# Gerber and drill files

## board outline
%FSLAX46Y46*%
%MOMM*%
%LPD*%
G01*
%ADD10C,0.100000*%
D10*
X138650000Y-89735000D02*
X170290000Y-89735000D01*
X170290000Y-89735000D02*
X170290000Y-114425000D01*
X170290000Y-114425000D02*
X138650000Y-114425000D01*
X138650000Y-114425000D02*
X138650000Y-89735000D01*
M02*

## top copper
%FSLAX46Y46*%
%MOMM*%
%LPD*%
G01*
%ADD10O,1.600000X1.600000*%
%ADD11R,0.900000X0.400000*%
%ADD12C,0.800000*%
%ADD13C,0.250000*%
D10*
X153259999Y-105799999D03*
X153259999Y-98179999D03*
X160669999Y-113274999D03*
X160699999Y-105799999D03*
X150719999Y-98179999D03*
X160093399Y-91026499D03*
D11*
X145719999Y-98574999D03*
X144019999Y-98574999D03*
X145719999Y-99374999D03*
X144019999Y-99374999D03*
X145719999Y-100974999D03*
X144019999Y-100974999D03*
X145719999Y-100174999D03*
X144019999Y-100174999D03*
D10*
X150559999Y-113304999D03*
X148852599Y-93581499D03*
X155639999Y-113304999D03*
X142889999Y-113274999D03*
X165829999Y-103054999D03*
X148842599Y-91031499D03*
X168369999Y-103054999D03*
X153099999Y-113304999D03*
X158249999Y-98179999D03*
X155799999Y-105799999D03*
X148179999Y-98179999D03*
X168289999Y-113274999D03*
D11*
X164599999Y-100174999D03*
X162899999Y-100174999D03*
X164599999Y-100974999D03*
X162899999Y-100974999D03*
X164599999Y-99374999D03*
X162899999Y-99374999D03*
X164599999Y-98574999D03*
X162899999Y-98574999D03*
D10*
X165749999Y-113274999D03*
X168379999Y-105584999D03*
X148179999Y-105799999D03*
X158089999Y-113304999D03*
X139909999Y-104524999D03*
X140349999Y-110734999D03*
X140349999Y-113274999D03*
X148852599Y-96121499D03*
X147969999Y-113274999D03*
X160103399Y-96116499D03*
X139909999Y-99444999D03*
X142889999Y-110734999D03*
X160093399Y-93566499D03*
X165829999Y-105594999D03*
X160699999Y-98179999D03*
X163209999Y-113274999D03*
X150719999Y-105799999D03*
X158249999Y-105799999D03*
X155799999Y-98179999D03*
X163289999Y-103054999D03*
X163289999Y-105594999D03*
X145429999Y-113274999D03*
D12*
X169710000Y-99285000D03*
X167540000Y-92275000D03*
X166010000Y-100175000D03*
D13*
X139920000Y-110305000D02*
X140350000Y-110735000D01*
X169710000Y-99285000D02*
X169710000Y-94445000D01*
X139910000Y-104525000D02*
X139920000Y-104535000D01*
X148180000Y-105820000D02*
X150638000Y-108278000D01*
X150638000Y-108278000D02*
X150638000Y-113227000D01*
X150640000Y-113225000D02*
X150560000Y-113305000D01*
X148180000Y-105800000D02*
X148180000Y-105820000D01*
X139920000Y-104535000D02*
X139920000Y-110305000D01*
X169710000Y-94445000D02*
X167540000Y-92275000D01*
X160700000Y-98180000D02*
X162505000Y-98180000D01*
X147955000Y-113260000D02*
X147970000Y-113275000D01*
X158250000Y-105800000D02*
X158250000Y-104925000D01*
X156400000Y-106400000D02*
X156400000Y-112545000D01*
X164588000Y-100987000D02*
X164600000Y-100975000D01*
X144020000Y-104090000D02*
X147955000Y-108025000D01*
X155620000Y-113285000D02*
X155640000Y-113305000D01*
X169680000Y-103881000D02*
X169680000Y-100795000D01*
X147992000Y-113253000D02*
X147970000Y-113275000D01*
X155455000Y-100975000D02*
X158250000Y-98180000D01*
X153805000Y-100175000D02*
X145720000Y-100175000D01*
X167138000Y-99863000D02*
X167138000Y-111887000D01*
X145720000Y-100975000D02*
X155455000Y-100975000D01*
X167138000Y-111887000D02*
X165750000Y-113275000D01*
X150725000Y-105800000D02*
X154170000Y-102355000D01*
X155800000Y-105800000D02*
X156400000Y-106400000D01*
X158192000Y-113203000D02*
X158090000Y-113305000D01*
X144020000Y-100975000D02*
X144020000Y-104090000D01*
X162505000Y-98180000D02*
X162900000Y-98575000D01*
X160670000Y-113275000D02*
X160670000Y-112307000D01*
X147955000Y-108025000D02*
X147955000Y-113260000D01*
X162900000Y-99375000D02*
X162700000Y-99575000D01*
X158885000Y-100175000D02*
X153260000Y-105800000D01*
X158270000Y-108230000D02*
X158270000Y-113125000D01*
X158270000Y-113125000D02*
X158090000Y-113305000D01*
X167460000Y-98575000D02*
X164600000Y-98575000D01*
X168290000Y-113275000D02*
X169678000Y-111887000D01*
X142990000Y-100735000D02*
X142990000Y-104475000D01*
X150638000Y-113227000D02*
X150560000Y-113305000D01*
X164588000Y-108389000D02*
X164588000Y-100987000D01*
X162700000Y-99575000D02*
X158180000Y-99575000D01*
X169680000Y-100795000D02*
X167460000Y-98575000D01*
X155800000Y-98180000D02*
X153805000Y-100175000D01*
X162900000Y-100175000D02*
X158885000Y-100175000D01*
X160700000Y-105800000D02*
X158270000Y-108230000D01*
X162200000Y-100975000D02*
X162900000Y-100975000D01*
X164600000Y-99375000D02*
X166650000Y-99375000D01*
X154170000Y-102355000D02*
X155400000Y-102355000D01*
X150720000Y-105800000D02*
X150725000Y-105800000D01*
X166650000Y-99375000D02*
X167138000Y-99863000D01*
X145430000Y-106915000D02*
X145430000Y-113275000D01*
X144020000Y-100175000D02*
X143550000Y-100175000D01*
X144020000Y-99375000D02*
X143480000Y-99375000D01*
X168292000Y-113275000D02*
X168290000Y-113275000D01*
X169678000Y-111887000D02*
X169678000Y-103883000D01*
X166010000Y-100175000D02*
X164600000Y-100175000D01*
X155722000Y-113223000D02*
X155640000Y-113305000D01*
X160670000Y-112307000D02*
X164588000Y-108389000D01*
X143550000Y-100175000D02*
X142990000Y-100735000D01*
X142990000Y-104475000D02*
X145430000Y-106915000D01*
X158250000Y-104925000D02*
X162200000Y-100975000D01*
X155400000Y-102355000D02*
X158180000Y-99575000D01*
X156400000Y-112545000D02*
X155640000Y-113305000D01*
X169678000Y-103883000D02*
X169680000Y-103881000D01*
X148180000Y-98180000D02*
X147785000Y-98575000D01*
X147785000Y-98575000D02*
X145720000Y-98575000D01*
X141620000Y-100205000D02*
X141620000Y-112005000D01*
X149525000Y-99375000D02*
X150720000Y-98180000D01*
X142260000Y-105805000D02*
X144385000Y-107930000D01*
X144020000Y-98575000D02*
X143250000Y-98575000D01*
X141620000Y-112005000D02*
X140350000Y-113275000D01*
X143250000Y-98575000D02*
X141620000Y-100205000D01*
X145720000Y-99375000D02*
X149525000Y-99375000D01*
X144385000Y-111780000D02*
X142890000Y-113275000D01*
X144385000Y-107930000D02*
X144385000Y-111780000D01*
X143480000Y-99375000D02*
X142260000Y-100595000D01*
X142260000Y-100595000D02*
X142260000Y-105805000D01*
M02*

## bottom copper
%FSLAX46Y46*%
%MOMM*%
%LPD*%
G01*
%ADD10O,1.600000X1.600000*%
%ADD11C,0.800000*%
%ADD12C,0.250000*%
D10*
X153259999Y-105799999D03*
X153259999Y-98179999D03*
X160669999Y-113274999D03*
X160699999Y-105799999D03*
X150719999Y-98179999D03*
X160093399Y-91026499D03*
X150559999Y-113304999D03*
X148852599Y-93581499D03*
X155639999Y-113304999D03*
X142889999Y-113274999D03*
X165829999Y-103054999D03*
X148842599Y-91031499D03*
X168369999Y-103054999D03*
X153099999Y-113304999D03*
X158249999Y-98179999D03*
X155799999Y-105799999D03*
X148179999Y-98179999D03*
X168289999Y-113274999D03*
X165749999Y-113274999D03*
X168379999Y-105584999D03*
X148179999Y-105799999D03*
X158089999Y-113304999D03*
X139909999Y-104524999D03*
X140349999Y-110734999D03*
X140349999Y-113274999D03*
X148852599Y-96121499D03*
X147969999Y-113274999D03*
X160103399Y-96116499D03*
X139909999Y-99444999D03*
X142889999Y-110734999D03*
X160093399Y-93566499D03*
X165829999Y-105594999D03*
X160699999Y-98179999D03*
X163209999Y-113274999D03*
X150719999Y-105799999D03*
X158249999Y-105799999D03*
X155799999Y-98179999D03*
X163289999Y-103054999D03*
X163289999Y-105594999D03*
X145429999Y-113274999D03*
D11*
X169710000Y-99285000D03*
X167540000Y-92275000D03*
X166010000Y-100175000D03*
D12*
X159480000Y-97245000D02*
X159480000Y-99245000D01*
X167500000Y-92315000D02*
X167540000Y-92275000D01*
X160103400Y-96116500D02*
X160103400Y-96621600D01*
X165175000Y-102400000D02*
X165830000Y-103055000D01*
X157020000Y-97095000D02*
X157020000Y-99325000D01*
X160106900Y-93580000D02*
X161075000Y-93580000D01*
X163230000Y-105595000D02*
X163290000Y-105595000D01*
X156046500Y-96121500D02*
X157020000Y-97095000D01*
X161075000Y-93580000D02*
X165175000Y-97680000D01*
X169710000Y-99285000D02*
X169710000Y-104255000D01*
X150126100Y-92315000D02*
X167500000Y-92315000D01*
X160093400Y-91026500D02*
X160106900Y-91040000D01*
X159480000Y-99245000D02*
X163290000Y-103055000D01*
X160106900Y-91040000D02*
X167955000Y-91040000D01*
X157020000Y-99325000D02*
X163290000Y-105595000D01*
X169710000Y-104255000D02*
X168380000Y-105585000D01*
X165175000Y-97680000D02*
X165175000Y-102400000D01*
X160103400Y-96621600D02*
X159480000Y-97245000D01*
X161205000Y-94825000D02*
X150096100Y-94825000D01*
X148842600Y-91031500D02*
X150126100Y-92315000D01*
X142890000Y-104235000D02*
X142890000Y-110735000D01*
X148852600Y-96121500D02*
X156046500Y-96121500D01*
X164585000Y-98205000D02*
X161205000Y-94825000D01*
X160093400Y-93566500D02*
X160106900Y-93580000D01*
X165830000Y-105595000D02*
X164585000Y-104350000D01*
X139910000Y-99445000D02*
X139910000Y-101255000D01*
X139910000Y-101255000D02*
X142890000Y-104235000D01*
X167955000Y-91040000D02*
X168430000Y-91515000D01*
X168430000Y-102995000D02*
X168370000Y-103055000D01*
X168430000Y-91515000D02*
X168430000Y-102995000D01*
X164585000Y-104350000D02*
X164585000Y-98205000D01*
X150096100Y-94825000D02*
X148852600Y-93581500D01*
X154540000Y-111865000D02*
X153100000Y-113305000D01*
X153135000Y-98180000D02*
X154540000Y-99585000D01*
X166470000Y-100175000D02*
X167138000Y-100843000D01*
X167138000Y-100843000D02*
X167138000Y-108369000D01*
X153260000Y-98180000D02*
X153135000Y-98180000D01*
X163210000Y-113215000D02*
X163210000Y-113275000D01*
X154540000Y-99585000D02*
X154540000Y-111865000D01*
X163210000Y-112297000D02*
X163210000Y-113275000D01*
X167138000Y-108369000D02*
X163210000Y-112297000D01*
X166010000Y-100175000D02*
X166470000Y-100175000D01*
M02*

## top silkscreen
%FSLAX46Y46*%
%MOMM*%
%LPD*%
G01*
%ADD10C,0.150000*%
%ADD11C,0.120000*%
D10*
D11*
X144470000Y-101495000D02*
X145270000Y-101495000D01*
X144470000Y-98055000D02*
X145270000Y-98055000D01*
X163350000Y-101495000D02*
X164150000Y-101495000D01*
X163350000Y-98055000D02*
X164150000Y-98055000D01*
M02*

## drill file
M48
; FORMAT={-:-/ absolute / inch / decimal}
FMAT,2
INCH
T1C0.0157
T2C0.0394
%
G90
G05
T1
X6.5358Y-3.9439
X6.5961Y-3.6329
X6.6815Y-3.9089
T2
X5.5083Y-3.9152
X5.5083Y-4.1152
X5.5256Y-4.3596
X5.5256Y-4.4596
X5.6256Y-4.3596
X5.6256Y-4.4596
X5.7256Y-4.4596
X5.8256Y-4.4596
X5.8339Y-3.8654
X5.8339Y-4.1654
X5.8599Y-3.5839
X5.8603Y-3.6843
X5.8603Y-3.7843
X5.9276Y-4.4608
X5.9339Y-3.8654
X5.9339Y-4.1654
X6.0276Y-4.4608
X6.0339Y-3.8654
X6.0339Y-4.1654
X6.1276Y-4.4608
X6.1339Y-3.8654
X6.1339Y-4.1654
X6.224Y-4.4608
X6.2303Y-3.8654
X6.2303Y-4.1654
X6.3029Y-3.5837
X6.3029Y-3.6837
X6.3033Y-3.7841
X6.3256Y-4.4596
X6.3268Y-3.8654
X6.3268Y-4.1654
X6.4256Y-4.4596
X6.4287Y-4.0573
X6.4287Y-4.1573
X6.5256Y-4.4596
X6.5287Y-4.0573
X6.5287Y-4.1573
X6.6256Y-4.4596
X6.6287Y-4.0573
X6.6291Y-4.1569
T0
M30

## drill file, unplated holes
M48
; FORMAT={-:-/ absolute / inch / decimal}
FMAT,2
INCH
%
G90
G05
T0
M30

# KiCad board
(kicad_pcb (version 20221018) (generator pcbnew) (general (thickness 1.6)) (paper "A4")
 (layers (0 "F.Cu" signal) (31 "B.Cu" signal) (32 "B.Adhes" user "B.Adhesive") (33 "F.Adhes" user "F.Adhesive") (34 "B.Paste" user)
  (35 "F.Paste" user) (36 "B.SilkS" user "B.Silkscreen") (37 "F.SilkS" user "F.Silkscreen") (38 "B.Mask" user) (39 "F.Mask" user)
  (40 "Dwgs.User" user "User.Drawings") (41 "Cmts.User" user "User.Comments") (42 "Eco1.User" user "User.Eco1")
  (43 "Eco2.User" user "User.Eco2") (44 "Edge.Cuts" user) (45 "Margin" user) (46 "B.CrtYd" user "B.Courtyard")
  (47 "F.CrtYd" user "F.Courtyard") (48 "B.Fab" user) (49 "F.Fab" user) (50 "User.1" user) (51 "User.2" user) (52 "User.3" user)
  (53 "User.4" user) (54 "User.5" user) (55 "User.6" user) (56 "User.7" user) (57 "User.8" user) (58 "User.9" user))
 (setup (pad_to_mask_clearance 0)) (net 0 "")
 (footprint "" (layer "F.Cu") (at 160.0934 93.5665 180)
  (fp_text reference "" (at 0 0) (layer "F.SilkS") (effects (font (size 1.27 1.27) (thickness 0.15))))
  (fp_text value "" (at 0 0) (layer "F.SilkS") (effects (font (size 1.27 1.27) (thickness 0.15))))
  (pad "12" thru_hole oval (at 0 0 90) (size 1.6 1.6) (drill 1) (layers "*.Cu" "*.Mask")))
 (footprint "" (layer "F.Cu") (at 142.89 113.275 90)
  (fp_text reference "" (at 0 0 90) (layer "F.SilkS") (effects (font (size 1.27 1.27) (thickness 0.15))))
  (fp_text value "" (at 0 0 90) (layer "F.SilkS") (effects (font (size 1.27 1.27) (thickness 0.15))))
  (pad "B" thru_hole oval (at 0 0 180) (size 1.6 1.6) (drill 1) (layers "*.Cu" "*.Mask")))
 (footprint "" (layer "F.Cu") (at 148.8526 96.1215)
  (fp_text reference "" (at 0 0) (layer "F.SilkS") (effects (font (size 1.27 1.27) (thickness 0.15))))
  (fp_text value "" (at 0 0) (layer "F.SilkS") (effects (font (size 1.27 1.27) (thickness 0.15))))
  (pad "10" thru_hole oval (at 0 0 270) (size 1.6 1.6) (drill 1) (layers "*.Cu" "*.Mask")))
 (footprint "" (layer "F.Cu") (at 150.56 113.305 -90)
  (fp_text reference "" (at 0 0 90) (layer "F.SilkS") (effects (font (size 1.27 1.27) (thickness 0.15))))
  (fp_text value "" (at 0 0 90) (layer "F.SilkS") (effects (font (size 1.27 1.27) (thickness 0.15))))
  (pad "4" thru_hole oval (at 0 0) (size 1.6 1.6) (drill 1) (layers "*.Cu" "*.Mask")))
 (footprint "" (layer "F.Cu") (at 140.35 110.725)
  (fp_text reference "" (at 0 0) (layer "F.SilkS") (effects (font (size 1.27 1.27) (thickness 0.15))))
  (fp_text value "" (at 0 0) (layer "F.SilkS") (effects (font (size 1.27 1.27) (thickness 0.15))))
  (pad "VCC" thru_hole oval (at 0 0.01 180) (size 1.6 1.6) (drill 1) (layers "*.Cu" "*.Mask")))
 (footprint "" (layer "F.Cu") (at 160.79 98.18 -90)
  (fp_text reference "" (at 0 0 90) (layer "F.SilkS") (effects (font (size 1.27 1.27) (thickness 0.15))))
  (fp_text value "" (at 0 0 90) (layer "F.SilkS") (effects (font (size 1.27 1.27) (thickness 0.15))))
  (pad "G" thru_hole oval (at 0 0.09) (size 1.6 1.6) (drill 1) (layers "*.Cu" "*.Mask")))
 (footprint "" (layer "F.Cu") (at 148.18 105.8)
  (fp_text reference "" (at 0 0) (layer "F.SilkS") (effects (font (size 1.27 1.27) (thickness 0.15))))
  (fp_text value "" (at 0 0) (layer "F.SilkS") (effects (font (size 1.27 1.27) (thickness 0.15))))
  (pad "4" thru_hole oval (at 0 0 90) (size 1.6 1.6) (drill 1) (layers "*.Cu" "*.Mask")))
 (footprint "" (layer "F.Cu") (at 155.64 113.305 -90)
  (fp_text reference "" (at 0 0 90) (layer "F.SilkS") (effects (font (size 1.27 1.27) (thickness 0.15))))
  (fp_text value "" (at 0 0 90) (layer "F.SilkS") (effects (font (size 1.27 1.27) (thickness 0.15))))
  (pad "2" thru_hole oval (at 0 0) (size 1.6 1.6) (drill 1) (layers "*.Cu" "*.Mask")))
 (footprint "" (layer "F.Cu") (at 165.75 113.275 90)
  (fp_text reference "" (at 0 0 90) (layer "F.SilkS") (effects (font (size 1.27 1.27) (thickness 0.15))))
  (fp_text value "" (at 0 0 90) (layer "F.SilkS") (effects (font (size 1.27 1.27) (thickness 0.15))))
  (pad "E" thru_hole oval (at 0 0 180) (size 1.6 1.6) (drill 1) (layers "*.Cu" "*.Mask")))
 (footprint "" (layer "F.Cu") (at 148.18 98.18 -90)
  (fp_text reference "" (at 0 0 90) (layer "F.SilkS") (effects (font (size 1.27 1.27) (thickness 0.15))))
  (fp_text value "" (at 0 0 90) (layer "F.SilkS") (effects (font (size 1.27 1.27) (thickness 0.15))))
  (pad "A" thru_hole oval (at 0 0) (size 1.6 1.6) (drill 1) (layers "*.Cu" "*.Mask")))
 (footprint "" (layer "F.Cu") (at 153.26 105.8 -90)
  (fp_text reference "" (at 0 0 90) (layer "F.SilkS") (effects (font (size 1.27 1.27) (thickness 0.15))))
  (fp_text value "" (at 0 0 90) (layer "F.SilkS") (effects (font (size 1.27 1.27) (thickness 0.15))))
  (pad "C" thru_hole oval (at 0 0) (size 1.6 1.6) (drill 1) (layers "*.Cu" "*.Mask")))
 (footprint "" (layer "F.Cu") (at 148.8426 91.0315)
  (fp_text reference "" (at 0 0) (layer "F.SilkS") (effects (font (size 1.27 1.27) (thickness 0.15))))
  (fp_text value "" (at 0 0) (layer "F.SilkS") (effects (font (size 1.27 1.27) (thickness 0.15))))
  (pad "V+" thru_hole oval (at 0 0 180) (size 1.6 1.6) (drill 1) (layers "*.Cu" "*.Mask")))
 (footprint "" (layer "F.Cu") (at 150.72 105.8 -90)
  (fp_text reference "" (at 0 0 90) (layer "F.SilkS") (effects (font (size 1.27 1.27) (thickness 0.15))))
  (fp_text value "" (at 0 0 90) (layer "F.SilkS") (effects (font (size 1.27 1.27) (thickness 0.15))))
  (pad "E" thru_hole oval (at 0 0) (size 1.6 1.6) (drill 1) (layers "*.Cu" "*.Mask")))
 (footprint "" (layer "F.Cu") (at 140.35 113.275 90)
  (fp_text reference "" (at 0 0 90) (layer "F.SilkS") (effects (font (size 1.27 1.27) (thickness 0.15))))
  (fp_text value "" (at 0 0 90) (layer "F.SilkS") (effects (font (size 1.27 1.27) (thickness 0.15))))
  (pad "A" thru_hole oval (at 0 0 180) (size 1.6 1.6) (drill 1) (layers "*.Cu" "*.Mask")))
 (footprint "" (layer "F.Cu") (at 163.29 103.055 90)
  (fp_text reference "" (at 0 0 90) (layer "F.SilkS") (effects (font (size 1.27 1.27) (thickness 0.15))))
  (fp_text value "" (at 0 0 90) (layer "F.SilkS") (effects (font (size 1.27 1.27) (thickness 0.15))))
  (pad "11" thru_hole oval (at 0 0 180) (size 1.6 1.6) (drill 1) (layers "*.Cu" "*.Mask")))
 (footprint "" (layer "F.Cu") (at 158.34 98.18 -90)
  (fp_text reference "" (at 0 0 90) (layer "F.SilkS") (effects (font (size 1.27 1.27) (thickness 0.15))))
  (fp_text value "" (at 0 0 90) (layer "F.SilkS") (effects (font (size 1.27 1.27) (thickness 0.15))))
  (pad "D" thru_hole oval (at 0 0.09) (size 1.6 1.6) (drill 1) (layers "*.Cu" "*.Mask")))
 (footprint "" (layer "F.Cu") (at 139.91 104.528 90)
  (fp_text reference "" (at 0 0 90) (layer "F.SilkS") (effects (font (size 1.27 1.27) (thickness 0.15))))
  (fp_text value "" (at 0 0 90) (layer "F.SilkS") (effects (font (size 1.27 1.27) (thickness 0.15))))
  (pad "VCC" thru_hole oval (at 0.003 0 90) (size 1.6 1.6) (drill 1) (layers "*.Cu" "*.Mask")))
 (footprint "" (layer "F.Cu") (at 145.43 113.275 90)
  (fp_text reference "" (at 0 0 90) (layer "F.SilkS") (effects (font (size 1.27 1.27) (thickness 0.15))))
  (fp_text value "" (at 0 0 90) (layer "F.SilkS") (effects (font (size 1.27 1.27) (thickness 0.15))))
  (pad "F" thru_hole oval (at 0 0 180) (size 1.6 1.6) (drill 1) (layers "*.Cu" "*.Mask")))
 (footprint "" (layer "F.Cu") (at 160.67 113.275 90)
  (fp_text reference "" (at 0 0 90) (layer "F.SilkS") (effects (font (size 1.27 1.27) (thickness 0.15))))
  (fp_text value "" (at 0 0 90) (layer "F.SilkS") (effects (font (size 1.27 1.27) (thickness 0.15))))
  (pad "DP" thru_hole oval (at 0 0 180) (size 1.6 1.6) (drill 1) (layers "*.Cu" "*.Mask")))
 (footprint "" (layer "F.Cu") (at 158.18 113.305 -90)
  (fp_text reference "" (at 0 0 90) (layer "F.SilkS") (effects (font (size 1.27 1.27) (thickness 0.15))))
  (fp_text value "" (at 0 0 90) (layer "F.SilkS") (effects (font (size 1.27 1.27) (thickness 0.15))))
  (pad "1" thru_hole oval (at 0 0.09) (size 1.6 1.6) (drill 1) (layers "*.Cu" "*.Mask")))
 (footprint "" (layer "F.Cu") (at 163.21 113.275 90)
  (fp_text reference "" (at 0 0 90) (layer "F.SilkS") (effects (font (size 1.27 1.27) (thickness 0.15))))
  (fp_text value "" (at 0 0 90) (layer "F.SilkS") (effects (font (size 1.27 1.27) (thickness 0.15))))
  (pad "C" thru_hole oval (at 0 0 180) (size 1.6 1.6) (drill 1) (layers "*.Cu" "*.Mask")))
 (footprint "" (layer "F.Cu") (at 150.72 98.18 -90)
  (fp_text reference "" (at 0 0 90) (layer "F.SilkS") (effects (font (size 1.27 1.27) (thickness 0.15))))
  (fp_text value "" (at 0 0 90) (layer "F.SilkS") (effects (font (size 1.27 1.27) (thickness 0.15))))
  (pad "B" thru_hole oval (at 0 0) (size 1.6 1.6) (drill 1) (layers "*.Cu" "*.Mask")))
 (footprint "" (layer "F.Cu") (at 139.91 99.448 90)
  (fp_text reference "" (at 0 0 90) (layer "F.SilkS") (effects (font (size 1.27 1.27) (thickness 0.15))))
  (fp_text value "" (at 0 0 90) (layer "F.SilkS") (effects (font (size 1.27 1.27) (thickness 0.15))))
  (pad "VCC" thru_hole oval (at 0.003 0 90) (size 1.6 1.6) (drill 1) (layers "*.Cu" "*.Mask")))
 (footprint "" (layer "F.Cu") (at 155.8 98.18 -90)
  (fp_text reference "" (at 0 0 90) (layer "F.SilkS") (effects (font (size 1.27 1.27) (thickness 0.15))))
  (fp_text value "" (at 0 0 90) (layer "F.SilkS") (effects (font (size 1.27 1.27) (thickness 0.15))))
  (pad "F" thru_hole oval (at 0 0) (size 1.6 1.6) (drill 1) (layers "*.Cu" "*.Mask")))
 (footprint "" (layer "F.Cu") (at 153.1 113.305 -90)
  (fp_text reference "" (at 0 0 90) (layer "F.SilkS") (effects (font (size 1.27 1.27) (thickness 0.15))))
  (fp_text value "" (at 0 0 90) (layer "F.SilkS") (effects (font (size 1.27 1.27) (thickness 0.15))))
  (pad "3" thru_hole oval (at 0 0) (size 1.6 1.6) (drill 1) (layers "*.Cu" "*.Mask")))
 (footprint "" (layer "F.Cu") (at 155.8 105.8 -90)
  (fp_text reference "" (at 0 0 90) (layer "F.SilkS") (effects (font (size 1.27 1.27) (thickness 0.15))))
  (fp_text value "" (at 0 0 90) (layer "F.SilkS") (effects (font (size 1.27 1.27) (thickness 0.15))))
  (pad "2" thru_hole oval (at 0 0) (size 1.6 1.6) (drill 1) (layers "*.Cu" "*.Mask")))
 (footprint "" (layer "F.Cu") (at 165.83 103.055 90)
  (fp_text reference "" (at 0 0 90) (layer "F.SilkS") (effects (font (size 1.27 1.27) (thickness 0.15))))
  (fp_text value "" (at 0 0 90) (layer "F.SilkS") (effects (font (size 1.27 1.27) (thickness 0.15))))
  (pad "12" thru_hole oval (at 0 0 180) (size 1.6 1.6) (drill 1) (layers "*.Cu" "*.Mask")))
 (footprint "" (layer "F.Cu") (at 160.79 105.8 -90)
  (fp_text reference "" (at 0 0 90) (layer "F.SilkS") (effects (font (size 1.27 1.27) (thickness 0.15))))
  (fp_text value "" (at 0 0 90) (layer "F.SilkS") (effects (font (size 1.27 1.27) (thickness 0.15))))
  (pad "1" thru_hole oval (at 0 0.09) (size 1.6 1.6) (drill 1) (layers "*.Cu" "*.Mask")))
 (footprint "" (layer "F.Cu") (at 160.0934 91.0265 180)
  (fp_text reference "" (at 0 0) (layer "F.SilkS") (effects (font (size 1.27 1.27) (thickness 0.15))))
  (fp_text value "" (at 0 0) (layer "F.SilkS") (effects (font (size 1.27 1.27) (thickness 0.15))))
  (pad "13" thru_hole oval (at 0 0 90) (size 1.6 1.6) (drill 1) (layers "*.Cu" "*.Mask")))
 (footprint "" (layer "F.Cu") (at 165.83 105.595 -90)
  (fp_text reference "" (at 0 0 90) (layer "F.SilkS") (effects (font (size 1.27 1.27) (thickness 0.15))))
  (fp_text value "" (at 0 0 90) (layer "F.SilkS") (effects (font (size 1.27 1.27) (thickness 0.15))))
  (pad "GND" thru_hole oval (at 0 0 180) (size 1.6 1.6) (drill 1) (layers "*.Cu" "*.Mask")))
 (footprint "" (layer "F.Cu") (at 153.26 98.18 -90)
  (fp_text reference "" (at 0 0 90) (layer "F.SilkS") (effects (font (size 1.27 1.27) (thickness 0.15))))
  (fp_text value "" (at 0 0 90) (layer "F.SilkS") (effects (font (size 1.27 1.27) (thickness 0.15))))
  (pad "3" thru_hole oval (at 0 0) (size 1.6 1.6) (drill 1) (layers "*.Cu" "*.Mask")))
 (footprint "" (layer "F.Cu") (at 142.89 110.735)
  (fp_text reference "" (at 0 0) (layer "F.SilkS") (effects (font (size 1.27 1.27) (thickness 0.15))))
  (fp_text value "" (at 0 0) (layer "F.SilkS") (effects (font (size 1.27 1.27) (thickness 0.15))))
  (pad "VCC" thru_hole oval (at 0 0 180) (size 1.6 1.6) (drill 1) (layers "*.Cu" "*.Mask")))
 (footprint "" (layer "F.Cu") (at 163.29 105.595 -90)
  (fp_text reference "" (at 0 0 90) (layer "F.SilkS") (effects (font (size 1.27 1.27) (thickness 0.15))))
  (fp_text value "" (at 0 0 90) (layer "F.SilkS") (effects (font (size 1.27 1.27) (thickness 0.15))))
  (pad "10" thru_hole oval (at 0 0 180) (size 1.6 1.6) (drill 1) (layers "*.Cu" "*.Mask")))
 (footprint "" (layer "F.Cu") (at 168.29 113.275 90)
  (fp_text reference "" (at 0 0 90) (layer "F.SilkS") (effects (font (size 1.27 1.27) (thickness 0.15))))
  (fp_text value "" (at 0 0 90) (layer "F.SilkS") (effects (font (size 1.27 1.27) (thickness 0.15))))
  (pad "G" thru_hole oval (at 0 0 180) (size 1.6 1.6) (drill 1) (layers "*.Cu" "*.Mask")))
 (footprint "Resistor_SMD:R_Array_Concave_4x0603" (layer "F.Cu") (at 163.75 99.775 180)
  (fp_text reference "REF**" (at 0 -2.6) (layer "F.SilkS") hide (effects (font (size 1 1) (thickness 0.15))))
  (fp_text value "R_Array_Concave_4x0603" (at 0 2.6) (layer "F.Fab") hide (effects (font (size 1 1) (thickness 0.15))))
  (fp_line (start 0.4 -1.72) (end -0.4 -1.72) (stroke (width 0.12) (type solid)) (layer "F.SilkS"))
  (fp_line (start 0.4 1.72) (end -0.4 1.72) (stroke (width 0.12) (type solid)) (layer "F.SilkS"))
  (pad "C" smd rect (at -0.85 -0.4 180) (size 0.9 0.4) (layers "F.Cu" "F.Paste" "F.Mask"))
  (pad "C" smd rect (at 0.85 -0.4 180) (size 0.9 0.4) (layers "F.Cu" "F.Paste" "F.Mask"))
  (pad "DP" smd rect (at -0.85 -1.2 180) (size 0.9 0.4) (layers "F.Cu" "F.Paste" "F.Mask"))
  (pad "DP" smd rect (at 0.85 -1.2 180) (size 0.9 0.4) (layers "F.Cu" "F.Paste" "F.Mask"))
  (pad "E" smd rect (at -0.85 0.4 180) (size 0.9 0.4) (layers "F.Cu" "F.Paste" "F.Mask"))
  (pad "E" smd rect (at 0.85 0.4 180) (size 0.9 0.4) (layers "F.Cu" "F.Paste" "F.Mask"))
  (pad "G" smd rect (at -0.85 1.2 180) (size 0.9 0.4) (layers "F.Cu" "F.Paste" "F.Mask"))
  (pad "G" smd rect (at 0.85 1.2 180) (size 0.9 0.4) (layers "F.Cu" "F.Paste" "F.Mask")))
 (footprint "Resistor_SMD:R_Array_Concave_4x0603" (layer "F.Cu") (at 144.87 99.775 180)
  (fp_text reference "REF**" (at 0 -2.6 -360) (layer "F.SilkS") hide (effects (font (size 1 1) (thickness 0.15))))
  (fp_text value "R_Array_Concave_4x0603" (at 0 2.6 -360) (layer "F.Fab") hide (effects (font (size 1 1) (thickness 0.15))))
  (fp_line (start 0.4 -1.72) (end -0.4 -1.72) (stroke (width 0.12) (type solid)) (layer "F.SilkS"))
  (fp_line (start 0.4 1.72) (end -0.4 1.72) (stroke (width 0.12) (type solid)) (layer "F.SilkS"))
  (pad "A" smd rect (at -0.85 1.2 180) (size 0.9 0.4) (layers "F.Cu" "F.Paste" "F.Mask"))
  (pad "A" smd rect (at 0.85 1.2 180) (size 0.9 0.4) (layers "F.Cu" "F.Paste" "F.Mask"))
  (pad "B" smd rect (at -0.85 0.4 180) (size 0.9 0.4) (layers "F.Cu" "F.Paste" "F.Mask"))
  (pad "B" smd rect (at 0.85 0.4 180) (size 0.9 0.4) (layers "F.Cu" "F.Paste" "F.Mask"))
  (pad "D" smd rect (at -0.85 -1.2 180) (size 0.9 0.4) (layers "F.Cu" "F.Paste" "F.Mask"))
  (pad "D" smd rect (at 0.85 -1.2 180) (size 0.9 0.4) (layers "F.Cu" "F.Paste" "F.Mask"))
  (pad "F" smd rect (at -0.85 -0.4 180) (size 0.9 0.4) (layers "F.Cu" "F.Paste" "F.Mask"))
  (pad "F" smd rect (at 0.85 -0.4 180) (size 0.9 0.4) (layers "F.Cu" "F.Paste" "F.Mask")))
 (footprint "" (layer "F.Cu") (at 168.37 103.055 180)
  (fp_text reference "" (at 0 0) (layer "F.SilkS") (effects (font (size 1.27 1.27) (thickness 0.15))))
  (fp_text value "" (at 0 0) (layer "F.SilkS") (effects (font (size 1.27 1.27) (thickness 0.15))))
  (pad "13" thru_hole oval (at 0 0 270) (size 1.6 1.6) (drill 1) (layers "*.Cu" "*.Mask")))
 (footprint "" (layer "F.Cu") (at 160.1034 96.1165 180)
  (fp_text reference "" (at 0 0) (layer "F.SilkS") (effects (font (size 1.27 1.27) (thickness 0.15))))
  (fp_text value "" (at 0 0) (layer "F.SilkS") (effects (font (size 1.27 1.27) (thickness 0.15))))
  (pad "11" thru_hole oval (at 0 0) (size 1.6 1.6) (drill 1) (layers "*.Cu" "*.Mask")))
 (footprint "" (layer "F.Cu") (at 158.34 105.8 -90)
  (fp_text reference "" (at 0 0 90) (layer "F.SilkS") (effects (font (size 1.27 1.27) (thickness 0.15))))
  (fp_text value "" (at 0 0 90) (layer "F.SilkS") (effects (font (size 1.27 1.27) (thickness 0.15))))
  (pad "DP" thru_hole oval (at 0 0.09) (size 1.6 1.6) (drill 1) (layers "*.Cu" "*.Mask")))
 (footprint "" (layer "F.Cu") (at 147.97 113.275 90)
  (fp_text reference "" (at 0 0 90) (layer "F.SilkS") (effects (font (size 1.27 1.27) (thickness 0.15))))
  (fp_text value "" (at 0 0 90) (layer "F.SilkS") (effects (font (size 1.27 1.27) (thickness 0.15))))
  (pad "D" thru_hole oval (at 0 0 180) (size 1.6 1.6) (drill 1) (layers "*.Cu" "*.Mask")))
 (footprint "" (layer "F.Cu") (at 148.8526 93.5815)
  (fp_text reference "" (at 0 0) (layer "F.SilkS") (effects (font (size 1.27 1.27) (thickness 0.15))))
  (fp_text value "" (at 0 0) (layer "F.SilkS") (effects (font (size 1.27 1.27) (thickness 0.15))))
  (pad "GND" thru_hole oval (at 0 0 270) (size 1.6 1.6) (drill 1) (layers "*.Cu" "*.Mask")))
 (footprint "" (layer "F.Cu") (at 168.38 105.585 -90)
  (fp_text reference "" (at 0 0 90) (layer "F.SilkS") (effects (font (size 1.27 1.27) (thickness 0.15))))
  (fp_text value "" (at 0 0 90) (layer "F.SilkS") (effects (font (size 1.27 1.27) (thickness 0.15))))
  (pad "V+" thru_hole oval (at 0 0 90) (size 1.6 1.6) (drill 1) (layers "*.Cu" "*.Mask")))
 (gr_rect (start 138.65 89.735) (end 170.29 114.425) (stroke (width 0.1) (type default)) (fill none) (layer "Edge.Cuts"))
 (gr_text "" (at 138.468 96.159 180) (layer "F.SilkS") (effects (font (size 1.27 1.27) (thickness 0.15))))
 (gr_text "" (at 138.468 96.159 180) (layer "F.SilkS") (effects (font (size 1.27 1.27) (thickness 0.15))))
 (segment (start 144.02 99.375) (end 143.48 99.375) (width 0.25) (layer "F.Cu") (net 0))
 (segment (start 139.91 104.525) (end 139.92 104.535) (width 0.25) (layer "F.Cu") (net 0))
 (segment (start 167.46 98.575) (end 164.6 98.575) (width 0.25) (layer "F.Cu") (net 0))
 (segment (start 169.71 99.285) (end 169.71 94.445) (width 0.25) (layer "F.Cu") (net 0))
 (segment (start 169.678 111.887) (end 169.678 103.883) (width 0.25) (layer "F.Cu") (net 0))
 (segment (start 150.725 105.8) (end 154.17 102.355) (width 0.25) (layer "F.Cu") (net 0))
 (segment (start 145.72 99.375) (end 149.525 99.375) (width 0.25) (layer "F.Cu") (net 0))
 (segment (start 155.62 113.285) (end 155.64 113.305) (width 0.25) (layer "F.Cu") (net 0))
 (segment (start 167.138 111.887) (end 165.75 113.275) (width 0.25) (layer "F.Cu") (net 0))
 (segment (start 147.785 98.575) (end 145.72 98.575) (width 0.25) (layer "F.Cu") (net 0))
 (segment (start 143.55 100.175) (end 142.99 100.735) (width 0.25) (layer "F.Cu") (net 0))
 (segment (start 150.64 113.225) (end 150.56 113.305) (width 0.25) (layer "F.Cu") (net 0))
 (segment (start 155.722 113.223) (end 155.64 113.305) (width 0.25) (layer "F.Cu") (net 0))
 (segment (start 164.6 99.375) (end 166.65 99.375) (width 0.25) (layer "F.Cu") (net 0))
 (segment (start 155.455 100.975) (end 158.25 98.18) (width 0.25) (layer "F.Cu") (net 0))
 (segment (start 143.48 99.375) (end 142.26 100.595) (width 0.25) (layer "F.Cu") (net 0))
 (segment (start 162.9 99.375) (end 162.7 99.575) (width 0.25) (layer "F.Cu") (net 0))
 (segment (start 156.4 112.545) (end 155.64 113.305) (width 0.25) (layer "F.Cu") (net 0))
 (segment (start 143.25 98.575) (end 141.62 100.205) (width 0.25) (layer "F.Cu") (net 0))
 (segment (start 144.385 107.93) (end 144.385 111.78) (width 0.25) (layer "F.Cu") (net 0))
 (segment (start 147.955 113.26) (end 147.97 113.275) (width 0.25) (layer "F.Cu") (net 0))
 (segment (start 169.68 103.881) (end 169.68 100.795) (width 0.25) (layer "F.Cu") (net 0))
 (segment (start 169.71 94.445) (end 167.54 92.275) (width 0.25) (layer "F.Cu") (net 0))
 (segment (start 142.99 100.735) (end 142.99 104.475) (width 0.25) (layer "F.Cu") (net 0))
 (segment (start 160.7 98.18) (end 162.505 98.18) (width 0.25) (layer "F.Cu") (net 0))
 (segment (start 141.62 100.205) (end 141.62 112.005) (width 0.25) (layer "F.Cu") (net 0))
 (segment (start 144.02 100.175) (end 143.55 100.175) (width 0.25) (layer "F.Cu") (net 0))
 (segment (start 150.638 113.227) (end 150.56 113.305) (width 0.25) (layer "F.Cu") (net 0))
 (segment (start 160.67 113.275) (end 160.67 112.307) (width 0.25) (layer "F.Cu") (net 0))
 (segment (start 139.92 104.535) (end 139.92 110.305) (width 0.25) (layer "F.Cu") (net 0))
 (segment (start 147.955 108.025) (end 147.955 113.26) (width 0.25) (layer "F.Cu") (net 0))
 (segment (start 155.8 98.18) (end 153.805 100.175) (width 0.25) (layer "F.Cu") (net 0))
 (segment (start 158.27 108.23) (end 158.27 113.125) (width 0.25) (layer "F.Cu") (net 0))
 (segment (start 148.18 105.82) (end 150.638 108.278) (width 0.25) (layer "F.Cu") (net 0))
 (segment (start 147.992 113.253) (end 147.97 113.275) (width 0.25) (layer "F.Cu") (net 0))
 (segment (start 169.678 103.883) (end 169.68 103.881) (width 0.25) (layer "F.Cu") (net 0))
 (segment (start 155.4 102.355) (end 158.18 99.575) (width 0.25) (layer "F.Cu") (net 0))
 (segment (start 156.4 106.4) (end 156.4 112.545) (width 0.25) (layer "F.Cu") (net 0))
 (segment (start 145.43 106.915) (end 145.43 113.275) (width 0.25) (layer "F.Cu") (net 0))
 (segment (start 160.67 112.307) (end 164.588 108.389) (width 0.25) (layer "F.Cu") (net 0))
 (segment (start 168.292 113.275) (end 168.29 113.275) (width 0.25) (layer "F.Cu") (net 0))
 (segment (start 141.62 112.005) (end 140.35 113.275) (width 0.25) (layer "F.Cu") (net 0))
 (segment (start 166.65 99.375) (end 167.138 99.863) (width 0.25) (layer "F.Cu") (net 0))
 (segment (start 150.638 108.278) (end 150.638 113.227) (width 0.25) (layer "F.Cu") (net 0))
 (segment (start 144.02 98.575) (end 143.25 98.575) (width 0.25) (layer "F.Cu") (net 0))
 (segment (start 144.02 104.09) (end 147.955 108.025) (width 0.25) (layer "F.Cu") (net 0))
 (segment (start 150.72 105.8) (end 150.725 105.8) (width 0.25) (layer "F.Cu") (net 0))
 (segment (start 162.9 100.175) (end 158.885 100.175) (width 0.25) (layer "F.Cu") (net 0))
 (segment (start 144.02 100.975) (end 144.02 104.09) (width 0.25) (layer "F.Cu") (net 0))
 (segment (start 164.588 100.987) (end 164.6 100.975) (width 0.25) (layer "F.Cu") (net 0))
 (segment (start 148.18 98.18) (end 147.785 98.575) (width 0.25) (layer "F.Cu") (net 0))
 (segment (start 158.25 104.925) (end 162.2 100.975) (width 0.25) (layer "F.Cu") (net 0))
 (segment (start 158.192 113.203) (end 158.09 113.305) (width 0.25) (layer "F.Cu") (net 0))
 (segment (start 167.138 99.863) (end 167.138 111.887) (width 0.25) (layer "F.Cu") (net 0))
 (segment (start 158.885 100.175) (end 153.26 105.8) (width 0.25) (layer "F.Cu") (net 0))
 (segment (start 160.7 105.8) (end 158.27 108.23) (width 0.25) (layer "F.Cu") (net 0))
 (segment (start 168.29 113.275) (end 169.678 111.887) (width 0.25) (layer "F.Cu") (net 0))
 (segment (start 148.18 105.8) (end 148.18 105.82) (width 0.25) (layer "F.Cu") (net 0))
 (segment (start 162.505 98.18) (end 162.9 98.575) (width 0.25) (layer "F.Cu") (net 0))
 (segment (start 155.8 105.8) (end 156.4 106.4) (width 0.25) (layer "F.Cu") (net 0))
 (segment (start 149.525 99.375) (end 150.72 98.18) (width 0.25) (layer "F.Cu") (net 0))
 (segment (start 158.25 105.8) (end 158.25 104.925) (width 0.25) (layer "F.Cu") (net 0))
 (segment (start 166.01 100.175) (end 164.6 100.175) (width 0.25) (layer "F.Cu") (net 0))
 (segment (start 162.2 100.975) (end 162.9 100.975) (width 0.25) (layer "F.Cu") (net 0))
 (segment (start 144.385 111.78) (end 142.89 113.275) (width 0.25) (layer "F.Cu") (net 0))
 (segment (start 153.805 100.175) (end 145.72 100.175) (width 0.25) (layer "F.Cu") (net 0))
 (segment (start 145.72 100.975) (end 155.455 100.975) (width 0.25) (layer "F.Cu") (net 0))
 (segment (start 139.92 110.305) (end 140.35 110.735) (width 0.25) (layer "F.Cu") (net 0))
 (segment (start 164.588 108.389) (end 164.588 100.987) (width 0.25) (layer "F.Cu") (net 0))
 (segment (start 158.27 113.125) (end 158.09 113.305) (width 0.25) (layer "F.Cu") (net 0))
 (segment (start 142.26 100.595) (end 142.26 105.805) (width 0.25) (layer "F.Cu") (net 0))
 (segment (start 154.17 102.355) (end 155.4 102.355) (width 0.25) (layer "F.Cu") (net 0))
 (segment (start 142.26 105.805) (end 144.385 107.93) (width 0.25) (layer "F.Cu") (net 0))
 (segment (start 142.99 104.475) (end 145.43 106.915) (width 0.25) (layer "F.Cu") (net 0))
 (segment (start 169.68 100.795) (end 167.46 98.575) (width 0.25) (layer "F.Cu") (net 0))
 (segment (start 162.7 99.575) (end 158.18 99.575) (width 0.25) (layer "F.Cu") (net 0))
 (via (at 167.54 92.275) (size 0.8) (drill 0.4) (layers "F.Cu" "B.Cu") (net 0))
 (via (at 166.01 100.175) (size 0.8) (drill 0.4) (layers "F.Cu" "B.Cu") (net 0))
 (via (at 169.71 99.285) (size 0.8) (drill 0.4) (layers "F.Cu" "B.Cu") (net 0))
 (segment (start 167.138 108.369) (end 163.21 112.297) (width 0.25) (layer "B.Cu") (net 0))
 (segment (start 160.0934 91.0265) (end 160.1069 91.04) (width 0.25) (layer "B.Cu") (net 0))
 (segment (start 157.02 99.325) (end 163.29 105.595) (width 0.25) (layer "B.Cu") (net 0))
 (segment (start 165.175 102.4) (end 165.83 103.055) (width 0.25) (layer "B.Cu") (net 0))
 (segment (start 167.955 91.04) (end 168.43 91.515) (width 0.25) (layer "B.Cu") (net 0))
 (segment (start 156.0465 96.1215) (end 157.02 97.095) (width 0.25) (layer "B.Cu") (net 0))
 (segment (start 159.48 99.245) (end 163.29 103.055) (width 0.25) (layer "B.Cu") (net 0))
 (segment (start 148.8426 91.0315) (end 150.1261 92.315) (width 0.25) (layer "B.Cu") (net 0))
 (segment (start 150.0961 94.825) (end 148.8526 93.5815) (width 0.25) (layer "B.Cu") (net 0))
 (segment (start 160.1069 93.58) (end 161.075 93.58) (width 0.25) (layer "B.Cu") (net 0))
 (segment (start 168.43 102.995) (end 168.37 103.055) (width 0.25) (layer "B.Cu") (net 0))
 (segment (start 167.5 92.315) (end 167.54 92.275) (width 0.25) (layer "B.Cu") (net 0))
 (segment (start 160.1034 96.1165) (end 160.1034 96.6216) (width 0.25) (layer "B.Cu") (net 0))
 (segment (start 160.1069 91.04) (end 167.955 91.04) (width 0.25) (layer "B.Cu") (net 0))
 (segment (start 164.585 104.35) (end 164.585 98.205) (width 0.25) (layer "B.Cu") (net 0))
 (segment (start 139.91 99.445) (end 139.91 101.255) (width 0.25) (layer "B.Cu") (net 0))
 (segment (start 168.43 91.515) (end 168.43 102.995) (width 0.25) (layer "B.Cu") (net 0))
 (segment (start 150.1261 92.315) (end 167.5 92.315) (width 0.25) (layer "B.Cu") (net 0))
 (segment (start 161.075 93.58) (end 165.175 97.68) (width 0.25) (layer "B.Cu") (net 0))
 (segment (start 153.135 98.18) (end 154.54 99.585) (width 0.25) (layer "B.Cu") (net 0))
 (segment (start 165.175 97.68) (end 165.175 102.4) (width 0.25) (layer "B.Cu") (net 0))
 (segment (start 165.83 105.595) (end 164.585 104.35) (width 0.25) (layer "B.Cu") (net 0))
 (segment (start 139.91 101.255) (end 142.89 104.235) (width 0.25) (layer "B.Cu") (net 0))
 (segment (start 142.89 104.235) (end 142.89 110.735) (width 0.25) (layer "B.Cu") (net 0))
 (segment (start 166.01 100.175) (end 166.47 100.175) (width 0.25) (layer "B.Cu") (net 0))
 (segment (start 157.02 97.095) (end 157.02 99.325) (width 0.25) (layer "B.Cu") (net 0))
 (segment (start 160.0934 93.5665) (end 160.1069 93.58) (width 0.25) (layer "B.Cu") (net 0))
 (segment (start 159.48 97.245) (end 159.48 99.245) (width 0.25) (layer "B.Cu") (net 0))
 (segment (start 163.23 105.595) (end 163.29 105.595) (width 0.25) (layer "B.Cu") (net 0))
 (segment (start 163.21 112.297) (end 163.21 113.275) (width 0.25) (layer "B.Cu") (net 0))
 (segment (start 166.47 100.175) (end 167.138 100.843) (width 0.25) (layer "B.Cu") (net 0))
 (segment (start 148.8526 96.1215) (end 156.0465 96.1215) (width 0.25) (layer "B.Cu") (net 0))
 (segment (start 154.54 111.865) (end 153.1 113.305) (width 0.25) (layer "B.Cu") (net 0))
 (segment (start 160.1034 96.6216) (end 159.48 97.245) (width 0.25) (layer "B.Cu") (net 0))
 (segment (start 163.21 113.215) (end 163.21 113.275) (width 0.25) (layer "B.Cu") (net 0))
 (segment (start 164.585 98.205) (end 161.205 94.825) (width 0.25) (layer "B.Cu") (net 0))
 (segment (start 161.205 94.825) (end 150.0961 94.825) (width 0.25) (layer "B.Cu") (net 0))
 (segment (start 153.26 98.18) (end 153.135 98.18) (width 0.25) (layer "B.Cu") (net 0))
 (segment (start 169.71 99.285) (end 169.71 104.255) (width 0.25) (layer "B.Cu") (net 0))
 (segment (start 167.138 100.843) (end 167.138 108.369) (width 0.25) (layer "B.Cu") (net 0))
 (segment (start 169.71 104.255) (end 168.38 105.585) (width 0.25) (layer "B.Cu") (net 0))
 (segment (start 154.54 99.585) (end 154.54 111.865) (width 0.25) (layer "B.Cu") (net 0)))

